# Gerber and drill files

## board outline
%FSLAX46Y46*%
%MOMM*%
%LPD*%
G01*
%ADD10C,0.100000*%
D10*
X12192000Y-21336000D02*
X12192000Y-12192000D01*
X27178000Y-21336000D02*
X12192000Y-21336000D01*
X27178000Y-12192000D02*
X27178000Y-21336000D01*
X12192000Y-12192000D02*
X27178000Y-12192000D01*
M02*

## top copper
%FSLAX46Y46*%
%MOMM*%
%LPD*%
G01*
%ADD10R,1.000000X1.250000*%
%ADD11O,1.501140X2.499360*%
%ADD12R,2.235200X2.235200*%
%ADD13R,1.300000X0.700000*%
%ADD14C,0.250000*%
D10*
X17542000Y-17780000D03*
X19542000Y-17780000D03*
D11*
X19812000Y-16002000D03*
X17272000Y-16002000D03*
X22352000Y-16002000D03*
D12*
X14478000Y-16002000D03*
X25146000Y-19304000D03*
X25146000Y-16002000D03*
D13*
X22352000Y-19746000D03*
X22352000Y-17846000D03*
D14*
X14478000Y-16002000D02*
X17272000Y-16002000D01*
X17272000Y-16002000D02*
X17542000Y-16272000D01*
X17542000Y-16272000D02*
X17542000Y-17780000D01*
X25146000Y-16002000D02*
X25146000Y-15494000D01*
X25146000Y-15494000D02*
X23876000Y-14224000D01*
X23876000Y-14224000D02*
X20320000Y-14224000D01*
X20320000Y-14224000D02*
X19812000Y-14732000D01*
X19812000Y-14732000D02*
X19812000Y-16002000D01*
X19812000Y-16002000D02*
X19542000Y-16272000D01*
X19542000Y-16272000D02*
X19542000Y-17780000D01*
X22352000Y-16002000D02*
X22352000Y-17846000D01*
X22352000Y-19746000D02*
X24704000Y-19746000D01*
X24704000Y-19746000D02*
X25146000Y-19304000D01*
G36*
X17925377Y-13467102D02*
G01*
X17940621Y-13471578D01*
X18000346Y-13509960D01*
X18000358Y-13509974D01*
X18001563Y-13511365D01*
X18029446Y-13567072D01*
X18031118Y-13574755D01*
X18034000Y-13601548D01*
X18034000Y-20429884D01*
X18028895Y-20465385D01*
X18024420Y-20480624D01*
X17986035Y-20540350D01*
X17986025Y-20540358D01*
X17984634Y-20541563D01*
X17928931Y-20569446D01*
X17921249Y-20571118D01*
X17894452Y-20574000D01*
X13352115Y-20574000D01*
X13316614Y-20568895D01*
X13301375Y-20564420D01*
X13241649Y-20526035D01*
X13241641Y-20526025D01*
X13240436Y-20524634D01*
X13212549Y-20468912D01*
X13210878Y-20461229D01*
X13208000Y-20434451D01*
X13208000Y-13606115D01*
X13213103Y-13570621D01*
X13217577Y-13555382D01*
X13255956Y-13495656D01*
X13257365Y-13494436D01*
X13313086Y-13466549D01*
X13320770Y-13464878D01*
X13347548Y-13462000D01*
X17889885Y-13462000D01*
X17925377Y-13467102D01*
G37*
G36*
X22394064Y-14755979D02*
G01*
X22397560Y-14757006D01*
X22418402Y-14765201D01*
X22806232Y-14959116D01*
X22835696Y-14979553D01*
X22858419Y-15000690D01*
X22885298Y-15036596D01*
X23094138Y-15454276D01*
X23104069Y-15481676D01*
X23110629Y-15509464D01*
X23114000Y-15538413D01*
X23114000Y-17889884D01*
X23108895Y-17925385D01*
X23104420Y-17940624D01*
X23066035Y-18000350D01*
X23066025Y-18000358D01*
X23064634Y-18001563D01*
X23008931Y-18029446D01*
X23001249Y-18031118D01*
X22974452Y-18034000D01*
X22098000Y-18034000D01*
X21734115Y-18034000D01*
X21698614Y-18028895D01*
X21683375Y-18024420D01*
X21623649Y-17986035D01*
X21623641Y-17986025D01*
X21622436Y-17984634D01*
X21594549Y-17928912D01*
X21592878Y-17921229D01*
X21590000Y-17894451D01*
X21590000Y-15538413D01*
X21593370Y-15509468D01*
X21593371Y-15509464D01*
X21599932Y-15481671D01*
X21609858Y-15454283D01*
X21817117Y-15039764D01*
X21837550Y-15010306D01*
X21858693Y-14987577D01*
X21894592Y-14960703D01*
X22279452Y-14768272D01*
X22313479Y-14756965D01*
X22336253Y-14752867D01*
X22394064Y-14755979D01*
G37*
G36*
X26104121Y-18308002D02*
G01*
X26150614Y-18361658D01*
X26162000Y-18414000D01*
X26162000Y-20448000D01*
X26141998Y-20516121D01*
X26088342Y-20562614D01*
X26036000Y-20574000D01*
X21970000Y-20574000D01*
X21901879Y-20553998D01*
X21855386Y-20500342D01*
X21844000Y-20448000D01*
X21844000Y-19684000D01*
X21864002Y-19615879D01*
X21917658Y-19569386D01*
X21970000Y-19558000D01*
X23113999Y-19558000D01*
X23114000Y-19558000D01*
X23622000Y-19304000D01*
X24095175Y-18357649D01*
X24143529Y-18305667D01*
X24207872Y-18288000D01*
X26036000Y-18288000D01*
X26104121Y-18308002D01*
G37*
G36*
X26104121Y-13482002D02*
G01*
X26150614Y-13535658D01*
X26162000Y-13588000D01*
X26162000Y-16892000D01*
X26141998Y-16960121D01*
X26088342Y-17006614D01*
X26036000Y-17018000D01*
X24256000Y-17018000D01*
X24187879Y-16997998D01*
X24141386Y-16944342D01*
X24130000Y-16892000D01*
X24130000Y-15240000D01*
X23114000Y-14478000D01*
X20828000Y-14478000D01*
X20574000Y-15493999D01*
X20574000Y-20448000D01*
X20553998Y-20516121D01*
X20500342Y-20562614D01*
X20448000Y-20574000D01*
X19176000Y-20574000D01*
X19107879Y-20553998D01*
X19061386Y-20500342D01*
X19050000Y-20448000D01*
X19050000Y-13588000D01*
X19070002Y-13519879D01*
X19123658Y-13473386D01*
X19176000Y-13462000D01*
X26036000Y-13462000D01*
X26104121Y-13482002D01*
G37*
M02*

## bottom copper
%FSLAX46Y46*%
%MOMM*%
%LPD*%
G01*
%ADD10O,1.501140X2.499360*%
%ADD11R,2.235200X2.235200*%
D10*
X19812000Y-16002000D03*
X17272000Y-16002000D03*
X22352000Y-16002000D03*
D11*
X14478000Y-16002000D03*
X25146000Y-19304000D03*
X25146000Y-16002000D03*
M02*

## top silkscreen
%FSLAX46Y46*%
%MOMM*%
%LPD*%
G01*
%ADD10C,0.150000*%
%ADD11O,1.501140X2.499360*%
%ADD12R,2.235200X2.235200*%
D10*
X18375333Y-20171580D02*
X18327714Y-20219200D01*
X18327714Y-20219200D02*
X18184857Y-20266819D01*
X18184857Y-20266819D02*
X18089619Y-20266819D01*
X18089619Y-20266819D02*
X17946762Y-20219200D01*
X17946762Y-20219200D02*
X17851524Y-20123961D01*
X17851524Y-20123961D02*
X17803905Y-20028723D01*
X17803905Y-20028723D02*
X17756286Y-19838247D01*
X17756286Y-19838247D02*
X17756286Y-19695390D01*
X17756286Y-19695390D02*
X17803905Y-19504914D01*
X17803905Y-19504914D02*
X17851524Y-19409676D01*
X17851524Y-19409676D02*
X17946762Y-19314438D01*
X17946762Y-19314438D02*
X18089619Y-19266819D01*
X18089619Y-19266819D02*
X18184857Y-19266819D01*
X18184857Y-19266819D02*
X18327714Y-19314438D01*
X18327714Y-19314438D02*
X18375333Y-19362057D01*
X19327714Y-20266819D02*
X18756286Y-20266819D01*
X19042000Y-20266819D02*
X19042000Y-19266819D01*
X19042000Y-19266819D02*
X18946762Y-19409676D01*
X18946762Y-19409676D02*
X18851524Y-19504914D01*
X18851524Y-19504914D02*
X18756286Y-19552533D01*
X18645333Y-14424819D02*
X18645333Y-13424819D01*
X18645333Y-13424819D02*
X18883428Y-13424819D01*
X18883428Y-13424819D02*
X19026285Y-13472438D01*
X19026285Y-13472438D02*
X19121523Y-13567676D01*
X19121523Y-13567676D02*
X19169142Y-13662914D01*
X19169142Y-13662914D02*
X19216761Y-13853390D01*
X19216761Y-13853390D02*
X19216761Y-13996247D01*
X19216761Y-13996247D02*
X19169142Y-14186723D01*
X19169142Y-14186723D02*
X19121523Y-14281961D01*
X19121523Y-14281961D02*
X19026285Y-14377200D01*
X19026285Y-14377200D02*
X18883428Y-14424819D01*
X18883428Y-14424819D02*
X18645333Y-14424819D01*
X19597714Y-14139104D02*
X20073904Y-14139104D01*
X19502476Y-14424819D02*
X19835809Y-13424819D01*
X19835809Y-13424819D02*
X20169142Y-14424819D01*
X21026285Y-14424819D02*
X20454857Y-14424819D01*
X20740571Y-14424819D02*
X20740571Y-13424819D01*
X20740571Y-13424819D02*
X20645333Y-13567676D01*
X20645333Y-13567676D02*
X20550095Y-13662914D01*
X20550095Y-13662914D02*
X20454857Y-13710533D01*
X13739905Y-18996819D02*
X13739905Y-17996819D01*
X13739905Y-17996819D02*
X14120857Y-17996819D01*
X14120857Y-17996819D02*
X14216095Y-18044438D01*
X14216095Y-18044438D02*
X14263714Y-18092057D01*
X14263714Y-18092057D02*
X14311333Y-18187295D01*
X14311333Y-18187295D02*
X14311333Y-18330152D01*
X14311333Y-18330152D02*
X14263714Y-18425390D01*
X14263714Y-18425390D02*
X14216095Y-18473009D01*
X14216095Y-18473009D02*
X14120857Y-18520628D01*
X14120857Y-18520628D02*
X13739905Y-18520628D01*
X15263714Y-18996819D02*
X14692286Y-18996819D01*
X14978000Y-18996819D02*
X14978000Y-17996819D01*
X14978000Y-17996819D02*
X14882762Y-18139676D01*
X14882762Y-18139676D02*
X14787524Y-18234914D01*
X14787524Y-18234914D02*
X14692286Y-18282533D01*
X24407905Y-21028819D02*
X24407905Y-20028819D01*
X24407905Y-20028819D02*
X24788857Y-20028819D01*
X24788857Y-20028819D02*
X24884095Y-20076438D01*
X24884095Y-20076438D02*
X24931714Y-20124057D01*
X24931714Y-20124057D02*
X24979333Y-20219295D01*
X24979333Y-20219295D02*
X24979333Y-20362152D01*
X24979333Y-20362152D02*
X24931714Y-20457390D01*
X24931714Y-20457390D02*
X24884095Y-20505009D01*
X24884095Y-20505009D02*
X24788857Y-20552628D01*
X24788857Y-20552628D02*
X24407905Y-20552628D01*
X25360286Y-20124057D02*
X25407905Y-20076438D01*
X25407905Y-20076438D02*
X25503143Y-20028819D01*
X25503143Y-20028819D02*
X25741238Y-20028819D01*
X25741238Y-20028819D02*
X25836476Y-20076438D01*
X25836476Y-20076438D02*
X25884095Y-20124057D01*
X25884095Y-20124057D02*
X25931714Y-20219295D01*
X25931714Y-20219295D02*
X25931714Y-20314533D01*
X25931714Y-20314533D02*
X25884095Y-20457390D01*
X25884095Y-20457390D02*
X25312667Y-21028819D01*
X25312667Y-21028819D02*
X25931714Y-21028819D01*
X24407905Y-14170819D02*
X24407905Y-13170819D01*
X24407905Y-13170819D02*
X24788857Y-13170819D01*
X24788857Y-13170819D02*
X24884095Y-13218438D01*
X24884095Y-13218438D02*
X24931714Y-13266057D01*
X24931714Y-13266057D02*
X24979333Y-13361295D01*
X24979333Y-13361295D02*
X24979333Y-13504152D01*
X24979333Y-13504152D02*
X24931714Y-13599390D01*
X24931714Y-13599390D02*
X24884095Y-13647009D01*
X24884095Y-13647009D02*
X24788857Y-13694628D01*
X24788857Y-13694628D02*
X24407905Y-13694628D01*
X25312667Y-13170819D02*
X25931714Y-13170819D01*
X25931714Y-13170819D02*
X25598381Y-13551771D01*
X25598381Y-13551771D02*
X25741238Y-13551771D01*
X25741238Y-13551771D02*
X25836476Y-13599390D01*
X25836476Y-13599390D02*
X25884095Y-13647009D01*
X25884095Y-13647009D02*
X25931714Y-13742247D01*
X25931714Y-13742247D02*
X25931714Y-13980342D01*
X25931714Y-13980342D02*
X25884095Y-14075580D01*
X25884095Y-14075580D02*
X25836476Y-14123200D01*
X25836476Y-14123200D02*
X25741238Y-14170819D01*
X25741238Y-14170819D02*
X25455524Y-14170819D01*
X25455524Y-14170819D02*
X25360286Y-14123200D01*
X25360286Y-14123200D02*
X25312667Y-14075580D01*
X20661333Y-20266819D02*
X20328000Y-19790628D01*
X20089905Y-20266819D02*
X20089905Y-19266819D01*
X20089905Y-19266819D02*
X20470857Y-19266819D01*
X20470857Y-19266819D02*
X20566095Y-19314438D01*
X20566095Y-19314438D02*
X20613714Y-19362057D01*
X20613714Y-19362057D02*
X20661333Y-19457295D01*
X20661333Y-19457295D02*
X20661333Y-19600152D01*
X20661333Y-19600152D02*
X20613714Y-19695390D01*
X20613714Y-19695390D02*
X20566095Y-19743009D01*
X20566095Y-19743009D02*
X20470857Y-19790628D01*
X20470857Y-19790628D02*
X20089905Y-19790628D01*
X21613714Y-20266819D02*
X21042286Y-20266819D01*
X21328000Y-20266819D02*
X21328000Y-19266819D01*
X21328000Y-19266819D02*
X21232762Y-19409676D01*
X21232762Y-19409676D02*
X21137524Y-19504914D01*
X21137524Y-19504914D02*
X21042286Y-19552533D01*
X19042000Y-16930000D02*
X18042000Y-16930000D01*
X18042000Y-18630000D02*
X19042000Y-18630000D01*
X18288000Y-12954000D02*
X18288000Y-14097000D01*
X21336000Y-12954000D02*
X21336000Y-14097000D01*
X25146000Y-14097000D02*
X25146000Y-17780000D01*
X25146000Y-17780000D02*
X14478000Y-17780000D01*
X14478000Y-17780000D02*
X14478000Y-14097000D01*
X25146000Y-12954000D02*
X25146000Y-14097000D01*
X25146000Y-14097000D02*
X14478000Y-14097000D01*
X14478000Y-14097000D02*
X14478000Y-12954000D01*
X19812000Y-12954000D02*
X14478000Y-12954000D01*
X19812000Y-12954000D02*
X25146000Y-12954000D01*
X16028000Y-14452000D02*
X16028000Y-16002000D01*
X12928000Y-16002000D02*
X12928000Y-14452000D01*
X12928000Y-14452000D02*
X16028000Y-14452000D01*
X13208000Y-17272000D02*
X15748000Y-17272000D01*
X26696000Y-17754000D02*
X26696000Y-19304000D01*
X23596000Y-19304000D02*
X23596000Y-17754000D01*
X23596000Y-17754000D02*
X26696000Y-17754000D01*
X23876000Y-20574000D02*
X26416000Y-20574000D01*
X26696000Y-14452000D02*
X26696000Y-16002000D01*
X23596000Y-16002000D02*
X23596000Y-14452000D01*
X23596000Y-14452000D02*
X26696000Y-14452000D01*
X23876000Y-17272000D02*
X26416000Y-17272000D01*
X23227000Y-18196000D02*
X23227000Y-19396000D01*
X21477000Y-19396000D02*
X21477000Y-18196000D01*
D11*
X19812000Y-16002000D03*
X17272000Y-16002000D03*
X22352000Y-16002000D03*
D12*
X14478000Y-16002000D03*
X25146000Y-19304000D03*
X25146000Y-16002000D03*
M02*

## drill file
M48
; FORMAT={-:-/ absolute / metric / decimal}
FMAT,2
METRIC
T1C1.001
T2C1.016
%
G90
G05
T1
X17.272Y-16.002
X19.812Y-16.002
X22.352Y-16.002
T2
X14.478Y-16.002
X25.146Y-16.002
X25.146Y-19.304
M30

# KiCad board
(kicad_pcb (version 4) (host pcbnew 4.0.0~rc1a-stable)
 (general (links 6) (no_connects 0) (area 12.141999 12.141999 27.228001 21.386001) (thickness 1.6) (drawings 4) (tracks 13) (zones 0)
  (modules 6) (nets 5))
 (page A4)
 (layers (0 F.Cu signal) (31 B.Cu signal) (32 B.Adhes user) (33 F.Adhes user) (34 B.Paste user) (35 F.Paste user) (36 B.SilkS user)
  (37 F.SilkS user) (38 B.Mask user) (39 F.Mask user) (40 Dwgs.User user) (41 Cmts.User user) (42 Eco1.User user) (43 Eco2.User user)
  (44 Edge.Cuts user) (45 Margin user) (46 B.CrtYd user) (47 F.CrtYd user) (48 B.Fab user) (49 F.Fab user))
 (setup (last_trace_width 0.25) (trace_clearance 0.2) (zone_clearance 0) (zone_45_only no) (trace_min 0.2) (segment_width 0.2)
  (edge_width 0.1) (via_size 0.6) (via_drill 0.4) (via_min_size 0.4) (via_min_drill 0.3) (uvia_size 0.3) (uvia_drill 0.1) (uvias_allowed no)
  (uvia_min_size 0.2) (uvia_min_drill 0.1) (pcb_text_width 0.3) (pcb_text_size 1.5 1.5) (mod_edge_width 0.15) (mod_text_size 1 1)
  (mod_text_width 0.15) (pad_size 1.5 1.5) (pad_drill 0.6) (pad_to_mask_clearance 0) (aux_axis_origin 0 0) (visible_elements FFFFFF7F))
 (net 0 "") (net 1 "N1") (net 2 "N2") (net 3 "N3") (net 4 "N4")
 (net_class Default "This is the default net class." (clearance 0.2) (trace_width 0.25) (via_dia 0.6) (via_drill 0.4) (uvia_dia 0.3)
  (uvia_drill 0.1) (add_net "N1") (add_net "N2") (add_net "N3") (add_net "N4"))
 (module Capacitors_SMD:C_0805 (layer F.Cu) (at 18.542 17.78)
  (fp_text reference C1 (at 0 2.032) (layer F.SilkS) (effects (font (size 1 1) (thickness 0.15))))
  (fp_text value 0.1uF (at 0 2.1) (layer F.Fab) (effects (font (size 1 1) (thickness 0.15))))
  (fp_line (start 0.5 -0.85) (end -0.5 -0.85) (layer F.SilkS) (width 0.15))
  (fp_line (start -0.5 0.85) (end 0.5 0.85) (layer F.SilkS) (width 0.15))
  (pad 1 smd rect (at -1 0) (size 1 1.25) (layers F.Cu F.Paste F.Mask) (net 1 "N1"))
  (pad 2 smd rect (at 1 0) (size 1 1.25) (layers F.Cu F.Paste F.Mask) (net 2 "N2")))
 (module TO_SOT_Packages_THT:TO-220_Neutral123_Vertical (layer F.Cu) (at 19.812 16.002)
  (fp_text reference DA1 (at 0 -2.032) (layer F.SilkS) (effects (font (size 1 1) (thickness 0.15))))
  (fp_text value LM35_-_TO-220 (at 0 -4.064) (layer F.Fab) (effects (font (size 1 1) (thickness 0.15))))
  (fp_line (start -1.524 -3.048) (end -1.524 -1.905) (layer F.SilkS) (width 0.15))
  (fp_line (start 1.524 -3.048) (end 1.524 -1.905) (layer F.SilkS) (width 0.15))
  (fp_line (start 5.334 -1.905) (end 5.334 1.778) (layer F.SilkS) (width 0.15))
  (fp_line (start 5.334 1.778) (end -5.334 1.778) (layer F.SilkS) (width 0.15))
  (fp_line (start -5.334 1.778) (end -5.334 -1.905) (layer F.SilkS) (width 0.15))
  (fp_line (start 5.334 -3.048) (end 5.334 -1.905) (layer F.SilkS) (width 0.15))
  (fp_line (start 5.334 -1.905) (end -5.334 -1.905) (layer F.SilkS) (width 0.15))
  (fp_line (start -5.334 -1.905) (end -5.334 -3.048) (layer F.SilkS) (width 0.15))
  (fp_line (start 0 -3.048) (end -5.334 -3.048) (layer F.SilkS) (width 0.15))
  (fp_line (start 0 -3.048) (end 5.334 -3.048) (layer F.SilkS) (width 0.15))
  (pad 2 thru_hole oval (at 0 0 90) (size 2.49936 1.50114) (drill 1.00076) (layers *.Cu *.Mask F.SilkS) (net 2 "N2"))
  (pad 1 thru_hole oval (at -2.54 0 90) (size 2.49936 1.50114) (drill 1.00076) (layers *.Cu *.Mask F.SilkS) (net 1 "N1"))
  (pad 3 thru_hole oval (at 2.54 0 90) (size 2.49936 1.50114) (drill 1.00076) (layers *.Cu *.Mask F.SilkS) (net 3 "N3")))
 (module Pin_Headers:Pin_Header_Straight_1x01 (layer F.Cu) (at 14.478 16.002)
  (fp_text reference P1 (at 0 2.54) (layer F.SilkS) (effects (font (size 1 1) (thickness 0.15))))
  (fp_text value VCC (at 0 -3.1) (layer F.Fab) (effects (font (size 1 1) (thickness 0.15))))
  (fp_line (start 1.55 -1.55) (end 1.55 0) (layer F.SilkS) (width 0.15))
  (fp_line (start -1.55 0) (end -1.55 -1.55) (layer F.SilkS) (width 0.15))
  (fp_line (start -1.55 -1.55) (end 1.55 -1.55) (layer F.SilkS) (width 0.15))
  (fp_line (start -1.27 1.27) (end 1.27 1.27) (layer F.SilkS) (width 0.15))
  (pad 1 thru_hole rect (at 0 0) (size 2.2352 2.2352) (drill 1.016) (layers *.Cu *.Mask F.SilkS) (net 1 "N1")))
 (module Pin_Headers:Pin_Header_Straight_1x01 (layer F.Cu) (at 25.146 19.304)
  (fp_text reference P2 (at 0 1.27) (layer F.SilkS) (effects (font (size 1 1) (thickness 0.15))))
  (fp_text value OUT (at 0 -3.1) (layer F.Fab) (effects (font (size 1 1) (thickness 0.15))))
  (fp_line (start 1.55 -1.55) (end 1.55 0) (layer F.SilkS) (width 0.15))
  (fp_line (start -1.55 0) (end -1.55 -1.55) (layer F.SilkS) (width 0.15))
  (fp_line (start -1.55 -1.55) (end 1.55 -1.55) (layer F.SilkS) (width 0.15))
  (fp_line (start -1.27 1.27) (end 1.27 1.27) (layer F.SilkS) (width 0.15))
  (pad 1 thru_hole rect (at 0 0) (size 2.2352 2.2352) (drill 1.016) (layers *.Cu *.Mask F.SilkS) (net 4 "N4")))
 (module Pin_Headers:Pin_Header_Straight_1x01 (layer F.Cu) (at 25.146 16.002)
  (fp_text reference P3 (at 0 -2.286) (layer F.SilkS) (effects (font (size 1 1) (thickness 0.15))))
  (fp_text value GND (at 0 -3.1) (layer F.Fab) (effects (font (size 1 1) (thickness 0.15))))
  (fp_line (start 1.55 -1.55) (end 1.55 0) (layer F.SilkS) (width 0.15))
  (fp_line (start -1.55 0) (end -1.55 -1.55) (layer F.SilkS) (width 0.15))
  (fp_line (start -1.55 -1.55) (end 1.55 -1.55) (layer F.SilkS) (width 0.15))
  (fp_line (start -1.27 1.27) (end 1.27 1.27) (layer F.SilkS) (width 0.15))
  (pad 1 thru_hole rect (at 0 0) (size 2.2352 2.2352) (drill 1.016) (layers *.Cu *.Mask F.SilkS) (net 2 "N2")))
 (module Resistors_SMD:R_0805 (layer F.Cu) (at 22.352 18.796 90)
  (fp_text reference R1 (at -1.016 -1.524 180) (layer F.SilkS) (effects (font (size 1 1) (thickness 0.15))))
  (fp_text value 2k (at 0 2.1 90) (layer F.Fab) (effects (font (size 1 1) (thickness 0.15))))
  (fp_line (start 0.6 0.875) (end -0.6 0.875) (layer F.SilkS) (width 0.15))
  (fp_line (start -0.6 -0.875) (end 0.6 -0.875) (layer F.SilkS) (width 0.15))
  (pad 1 smd rect (at -0.95 0 90) (size 0.7 1.3) (layers F.Cu F.Paste F.Mask) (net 4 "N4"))
  (pad 2 smd rect (at 0.95 0 90) (size 0.7 1.3) (layers F.Cu F.Paste F.Mask) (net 3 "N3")))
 (gr_line (start 12.192 21.336) (end 12.192 12.192) (angle 90) (layer Edge.Cuts) (width 0.1))
 (gr_line (start 27.178 21.336) (end 12.192 21.336) (angle 90) (layer Edge.Cuts) (width 0.1))
 (gr_line (start 27.178 12.192) (end 27.178 21.336) (angle 90) (layer Edge.Cuts) (width 0.1))
 (gr_line (start 12.192 12.192) (end 27.178 12.192) (angle 90) (layer Edge.Cuts) (width 0.1))
 (segment (start 14.478 16.002) (end 17.272 16.002) (width 0.25) (layer F.Cu) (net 1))
 (segment (start 17.272 16.002) (end 17.542 16.272) (width 0.25) (layer F.Cu) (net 1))
 (segment (start 17.542 16.272) (end 17.542 17.78) (width 0.25) (layer F.Cu) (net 1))
 (segment (start 25.146 16.002) (end 25.146 15.494) (width 0.25) (layer F.Cu) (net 2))
 (segment (start 25.146 15.494) (end 23.876 14.224) (width 0.25) (layer F.Cu) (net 2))
 (segment (start 23.876 14.224) (end 20.32 14.224) (width 0.25) (layer F.Cu) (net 2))
 (segment (start 20.32 14.224) (end 19.812 14.732) (width 0.25) (layer F.Cu) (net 2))
 (segment (start 19.812 14.732) (end 19.812 16.002) (width 0.25) (layer F.Cu) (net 2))
 (segment (start 19.812 16.002) (end 19.542 16.272) (width 0.25) (layer F.Cu) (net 2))
 (segment (start 19.542 16.272) (end 19.542 17.78) (width 0.25) (layer F.Cu) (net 2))
 (segment (start 22.352 16.002) (end 22.352 17.846) (width 0.25) (layer F.Cu) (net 3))
 (segment (start 22.352 19.746) (end 24.704 19.746) (width 0.25) (layer F.Cu) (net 4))
 (segment (start 24.704 19.746) (end 25.146 19.304) (width 0.25) (layer F.Cu) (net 4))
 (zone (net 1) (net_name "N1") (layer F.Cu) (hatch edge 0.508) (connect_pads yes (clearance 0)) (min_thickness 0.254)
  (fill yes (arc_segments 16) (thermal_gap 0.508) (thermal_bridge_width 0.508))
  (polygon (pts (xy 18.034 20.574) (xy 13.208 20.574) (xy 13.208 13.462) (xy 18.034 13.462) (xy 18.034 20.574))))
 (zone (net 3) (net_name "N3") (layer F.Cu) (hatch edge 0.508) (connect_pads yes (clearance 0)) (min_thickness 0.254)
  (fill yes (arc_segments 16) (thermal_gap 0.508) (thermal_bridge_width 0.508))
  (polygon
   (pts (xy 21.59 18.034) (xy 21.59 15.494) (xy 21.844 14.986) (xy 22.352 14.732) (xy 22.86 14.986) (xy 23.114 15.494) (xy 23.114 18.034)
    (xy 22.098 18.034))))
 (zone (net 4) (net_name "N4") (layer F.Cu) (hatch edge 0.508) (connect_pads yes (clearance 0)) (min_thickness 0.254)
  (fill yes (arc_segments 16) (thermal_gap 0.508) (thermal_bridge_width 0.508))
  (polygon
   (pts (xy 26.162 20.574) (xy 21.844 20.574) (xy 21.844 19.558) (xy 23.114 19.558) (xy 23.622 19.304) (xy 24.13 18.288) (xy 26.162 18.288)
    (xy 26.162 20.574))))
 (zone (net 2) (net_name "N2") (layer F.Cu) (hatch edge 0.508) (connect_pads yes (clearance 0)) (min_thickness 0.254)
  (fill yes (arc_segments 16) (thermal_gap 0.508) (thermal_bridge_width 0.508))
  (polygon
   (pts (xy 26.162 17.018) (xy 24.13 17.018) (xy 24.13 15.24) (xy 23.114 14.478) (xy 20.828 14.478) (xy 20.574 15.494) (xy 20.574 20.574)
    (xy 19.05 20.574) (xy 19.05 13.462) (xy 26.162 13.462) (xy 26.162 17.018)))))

